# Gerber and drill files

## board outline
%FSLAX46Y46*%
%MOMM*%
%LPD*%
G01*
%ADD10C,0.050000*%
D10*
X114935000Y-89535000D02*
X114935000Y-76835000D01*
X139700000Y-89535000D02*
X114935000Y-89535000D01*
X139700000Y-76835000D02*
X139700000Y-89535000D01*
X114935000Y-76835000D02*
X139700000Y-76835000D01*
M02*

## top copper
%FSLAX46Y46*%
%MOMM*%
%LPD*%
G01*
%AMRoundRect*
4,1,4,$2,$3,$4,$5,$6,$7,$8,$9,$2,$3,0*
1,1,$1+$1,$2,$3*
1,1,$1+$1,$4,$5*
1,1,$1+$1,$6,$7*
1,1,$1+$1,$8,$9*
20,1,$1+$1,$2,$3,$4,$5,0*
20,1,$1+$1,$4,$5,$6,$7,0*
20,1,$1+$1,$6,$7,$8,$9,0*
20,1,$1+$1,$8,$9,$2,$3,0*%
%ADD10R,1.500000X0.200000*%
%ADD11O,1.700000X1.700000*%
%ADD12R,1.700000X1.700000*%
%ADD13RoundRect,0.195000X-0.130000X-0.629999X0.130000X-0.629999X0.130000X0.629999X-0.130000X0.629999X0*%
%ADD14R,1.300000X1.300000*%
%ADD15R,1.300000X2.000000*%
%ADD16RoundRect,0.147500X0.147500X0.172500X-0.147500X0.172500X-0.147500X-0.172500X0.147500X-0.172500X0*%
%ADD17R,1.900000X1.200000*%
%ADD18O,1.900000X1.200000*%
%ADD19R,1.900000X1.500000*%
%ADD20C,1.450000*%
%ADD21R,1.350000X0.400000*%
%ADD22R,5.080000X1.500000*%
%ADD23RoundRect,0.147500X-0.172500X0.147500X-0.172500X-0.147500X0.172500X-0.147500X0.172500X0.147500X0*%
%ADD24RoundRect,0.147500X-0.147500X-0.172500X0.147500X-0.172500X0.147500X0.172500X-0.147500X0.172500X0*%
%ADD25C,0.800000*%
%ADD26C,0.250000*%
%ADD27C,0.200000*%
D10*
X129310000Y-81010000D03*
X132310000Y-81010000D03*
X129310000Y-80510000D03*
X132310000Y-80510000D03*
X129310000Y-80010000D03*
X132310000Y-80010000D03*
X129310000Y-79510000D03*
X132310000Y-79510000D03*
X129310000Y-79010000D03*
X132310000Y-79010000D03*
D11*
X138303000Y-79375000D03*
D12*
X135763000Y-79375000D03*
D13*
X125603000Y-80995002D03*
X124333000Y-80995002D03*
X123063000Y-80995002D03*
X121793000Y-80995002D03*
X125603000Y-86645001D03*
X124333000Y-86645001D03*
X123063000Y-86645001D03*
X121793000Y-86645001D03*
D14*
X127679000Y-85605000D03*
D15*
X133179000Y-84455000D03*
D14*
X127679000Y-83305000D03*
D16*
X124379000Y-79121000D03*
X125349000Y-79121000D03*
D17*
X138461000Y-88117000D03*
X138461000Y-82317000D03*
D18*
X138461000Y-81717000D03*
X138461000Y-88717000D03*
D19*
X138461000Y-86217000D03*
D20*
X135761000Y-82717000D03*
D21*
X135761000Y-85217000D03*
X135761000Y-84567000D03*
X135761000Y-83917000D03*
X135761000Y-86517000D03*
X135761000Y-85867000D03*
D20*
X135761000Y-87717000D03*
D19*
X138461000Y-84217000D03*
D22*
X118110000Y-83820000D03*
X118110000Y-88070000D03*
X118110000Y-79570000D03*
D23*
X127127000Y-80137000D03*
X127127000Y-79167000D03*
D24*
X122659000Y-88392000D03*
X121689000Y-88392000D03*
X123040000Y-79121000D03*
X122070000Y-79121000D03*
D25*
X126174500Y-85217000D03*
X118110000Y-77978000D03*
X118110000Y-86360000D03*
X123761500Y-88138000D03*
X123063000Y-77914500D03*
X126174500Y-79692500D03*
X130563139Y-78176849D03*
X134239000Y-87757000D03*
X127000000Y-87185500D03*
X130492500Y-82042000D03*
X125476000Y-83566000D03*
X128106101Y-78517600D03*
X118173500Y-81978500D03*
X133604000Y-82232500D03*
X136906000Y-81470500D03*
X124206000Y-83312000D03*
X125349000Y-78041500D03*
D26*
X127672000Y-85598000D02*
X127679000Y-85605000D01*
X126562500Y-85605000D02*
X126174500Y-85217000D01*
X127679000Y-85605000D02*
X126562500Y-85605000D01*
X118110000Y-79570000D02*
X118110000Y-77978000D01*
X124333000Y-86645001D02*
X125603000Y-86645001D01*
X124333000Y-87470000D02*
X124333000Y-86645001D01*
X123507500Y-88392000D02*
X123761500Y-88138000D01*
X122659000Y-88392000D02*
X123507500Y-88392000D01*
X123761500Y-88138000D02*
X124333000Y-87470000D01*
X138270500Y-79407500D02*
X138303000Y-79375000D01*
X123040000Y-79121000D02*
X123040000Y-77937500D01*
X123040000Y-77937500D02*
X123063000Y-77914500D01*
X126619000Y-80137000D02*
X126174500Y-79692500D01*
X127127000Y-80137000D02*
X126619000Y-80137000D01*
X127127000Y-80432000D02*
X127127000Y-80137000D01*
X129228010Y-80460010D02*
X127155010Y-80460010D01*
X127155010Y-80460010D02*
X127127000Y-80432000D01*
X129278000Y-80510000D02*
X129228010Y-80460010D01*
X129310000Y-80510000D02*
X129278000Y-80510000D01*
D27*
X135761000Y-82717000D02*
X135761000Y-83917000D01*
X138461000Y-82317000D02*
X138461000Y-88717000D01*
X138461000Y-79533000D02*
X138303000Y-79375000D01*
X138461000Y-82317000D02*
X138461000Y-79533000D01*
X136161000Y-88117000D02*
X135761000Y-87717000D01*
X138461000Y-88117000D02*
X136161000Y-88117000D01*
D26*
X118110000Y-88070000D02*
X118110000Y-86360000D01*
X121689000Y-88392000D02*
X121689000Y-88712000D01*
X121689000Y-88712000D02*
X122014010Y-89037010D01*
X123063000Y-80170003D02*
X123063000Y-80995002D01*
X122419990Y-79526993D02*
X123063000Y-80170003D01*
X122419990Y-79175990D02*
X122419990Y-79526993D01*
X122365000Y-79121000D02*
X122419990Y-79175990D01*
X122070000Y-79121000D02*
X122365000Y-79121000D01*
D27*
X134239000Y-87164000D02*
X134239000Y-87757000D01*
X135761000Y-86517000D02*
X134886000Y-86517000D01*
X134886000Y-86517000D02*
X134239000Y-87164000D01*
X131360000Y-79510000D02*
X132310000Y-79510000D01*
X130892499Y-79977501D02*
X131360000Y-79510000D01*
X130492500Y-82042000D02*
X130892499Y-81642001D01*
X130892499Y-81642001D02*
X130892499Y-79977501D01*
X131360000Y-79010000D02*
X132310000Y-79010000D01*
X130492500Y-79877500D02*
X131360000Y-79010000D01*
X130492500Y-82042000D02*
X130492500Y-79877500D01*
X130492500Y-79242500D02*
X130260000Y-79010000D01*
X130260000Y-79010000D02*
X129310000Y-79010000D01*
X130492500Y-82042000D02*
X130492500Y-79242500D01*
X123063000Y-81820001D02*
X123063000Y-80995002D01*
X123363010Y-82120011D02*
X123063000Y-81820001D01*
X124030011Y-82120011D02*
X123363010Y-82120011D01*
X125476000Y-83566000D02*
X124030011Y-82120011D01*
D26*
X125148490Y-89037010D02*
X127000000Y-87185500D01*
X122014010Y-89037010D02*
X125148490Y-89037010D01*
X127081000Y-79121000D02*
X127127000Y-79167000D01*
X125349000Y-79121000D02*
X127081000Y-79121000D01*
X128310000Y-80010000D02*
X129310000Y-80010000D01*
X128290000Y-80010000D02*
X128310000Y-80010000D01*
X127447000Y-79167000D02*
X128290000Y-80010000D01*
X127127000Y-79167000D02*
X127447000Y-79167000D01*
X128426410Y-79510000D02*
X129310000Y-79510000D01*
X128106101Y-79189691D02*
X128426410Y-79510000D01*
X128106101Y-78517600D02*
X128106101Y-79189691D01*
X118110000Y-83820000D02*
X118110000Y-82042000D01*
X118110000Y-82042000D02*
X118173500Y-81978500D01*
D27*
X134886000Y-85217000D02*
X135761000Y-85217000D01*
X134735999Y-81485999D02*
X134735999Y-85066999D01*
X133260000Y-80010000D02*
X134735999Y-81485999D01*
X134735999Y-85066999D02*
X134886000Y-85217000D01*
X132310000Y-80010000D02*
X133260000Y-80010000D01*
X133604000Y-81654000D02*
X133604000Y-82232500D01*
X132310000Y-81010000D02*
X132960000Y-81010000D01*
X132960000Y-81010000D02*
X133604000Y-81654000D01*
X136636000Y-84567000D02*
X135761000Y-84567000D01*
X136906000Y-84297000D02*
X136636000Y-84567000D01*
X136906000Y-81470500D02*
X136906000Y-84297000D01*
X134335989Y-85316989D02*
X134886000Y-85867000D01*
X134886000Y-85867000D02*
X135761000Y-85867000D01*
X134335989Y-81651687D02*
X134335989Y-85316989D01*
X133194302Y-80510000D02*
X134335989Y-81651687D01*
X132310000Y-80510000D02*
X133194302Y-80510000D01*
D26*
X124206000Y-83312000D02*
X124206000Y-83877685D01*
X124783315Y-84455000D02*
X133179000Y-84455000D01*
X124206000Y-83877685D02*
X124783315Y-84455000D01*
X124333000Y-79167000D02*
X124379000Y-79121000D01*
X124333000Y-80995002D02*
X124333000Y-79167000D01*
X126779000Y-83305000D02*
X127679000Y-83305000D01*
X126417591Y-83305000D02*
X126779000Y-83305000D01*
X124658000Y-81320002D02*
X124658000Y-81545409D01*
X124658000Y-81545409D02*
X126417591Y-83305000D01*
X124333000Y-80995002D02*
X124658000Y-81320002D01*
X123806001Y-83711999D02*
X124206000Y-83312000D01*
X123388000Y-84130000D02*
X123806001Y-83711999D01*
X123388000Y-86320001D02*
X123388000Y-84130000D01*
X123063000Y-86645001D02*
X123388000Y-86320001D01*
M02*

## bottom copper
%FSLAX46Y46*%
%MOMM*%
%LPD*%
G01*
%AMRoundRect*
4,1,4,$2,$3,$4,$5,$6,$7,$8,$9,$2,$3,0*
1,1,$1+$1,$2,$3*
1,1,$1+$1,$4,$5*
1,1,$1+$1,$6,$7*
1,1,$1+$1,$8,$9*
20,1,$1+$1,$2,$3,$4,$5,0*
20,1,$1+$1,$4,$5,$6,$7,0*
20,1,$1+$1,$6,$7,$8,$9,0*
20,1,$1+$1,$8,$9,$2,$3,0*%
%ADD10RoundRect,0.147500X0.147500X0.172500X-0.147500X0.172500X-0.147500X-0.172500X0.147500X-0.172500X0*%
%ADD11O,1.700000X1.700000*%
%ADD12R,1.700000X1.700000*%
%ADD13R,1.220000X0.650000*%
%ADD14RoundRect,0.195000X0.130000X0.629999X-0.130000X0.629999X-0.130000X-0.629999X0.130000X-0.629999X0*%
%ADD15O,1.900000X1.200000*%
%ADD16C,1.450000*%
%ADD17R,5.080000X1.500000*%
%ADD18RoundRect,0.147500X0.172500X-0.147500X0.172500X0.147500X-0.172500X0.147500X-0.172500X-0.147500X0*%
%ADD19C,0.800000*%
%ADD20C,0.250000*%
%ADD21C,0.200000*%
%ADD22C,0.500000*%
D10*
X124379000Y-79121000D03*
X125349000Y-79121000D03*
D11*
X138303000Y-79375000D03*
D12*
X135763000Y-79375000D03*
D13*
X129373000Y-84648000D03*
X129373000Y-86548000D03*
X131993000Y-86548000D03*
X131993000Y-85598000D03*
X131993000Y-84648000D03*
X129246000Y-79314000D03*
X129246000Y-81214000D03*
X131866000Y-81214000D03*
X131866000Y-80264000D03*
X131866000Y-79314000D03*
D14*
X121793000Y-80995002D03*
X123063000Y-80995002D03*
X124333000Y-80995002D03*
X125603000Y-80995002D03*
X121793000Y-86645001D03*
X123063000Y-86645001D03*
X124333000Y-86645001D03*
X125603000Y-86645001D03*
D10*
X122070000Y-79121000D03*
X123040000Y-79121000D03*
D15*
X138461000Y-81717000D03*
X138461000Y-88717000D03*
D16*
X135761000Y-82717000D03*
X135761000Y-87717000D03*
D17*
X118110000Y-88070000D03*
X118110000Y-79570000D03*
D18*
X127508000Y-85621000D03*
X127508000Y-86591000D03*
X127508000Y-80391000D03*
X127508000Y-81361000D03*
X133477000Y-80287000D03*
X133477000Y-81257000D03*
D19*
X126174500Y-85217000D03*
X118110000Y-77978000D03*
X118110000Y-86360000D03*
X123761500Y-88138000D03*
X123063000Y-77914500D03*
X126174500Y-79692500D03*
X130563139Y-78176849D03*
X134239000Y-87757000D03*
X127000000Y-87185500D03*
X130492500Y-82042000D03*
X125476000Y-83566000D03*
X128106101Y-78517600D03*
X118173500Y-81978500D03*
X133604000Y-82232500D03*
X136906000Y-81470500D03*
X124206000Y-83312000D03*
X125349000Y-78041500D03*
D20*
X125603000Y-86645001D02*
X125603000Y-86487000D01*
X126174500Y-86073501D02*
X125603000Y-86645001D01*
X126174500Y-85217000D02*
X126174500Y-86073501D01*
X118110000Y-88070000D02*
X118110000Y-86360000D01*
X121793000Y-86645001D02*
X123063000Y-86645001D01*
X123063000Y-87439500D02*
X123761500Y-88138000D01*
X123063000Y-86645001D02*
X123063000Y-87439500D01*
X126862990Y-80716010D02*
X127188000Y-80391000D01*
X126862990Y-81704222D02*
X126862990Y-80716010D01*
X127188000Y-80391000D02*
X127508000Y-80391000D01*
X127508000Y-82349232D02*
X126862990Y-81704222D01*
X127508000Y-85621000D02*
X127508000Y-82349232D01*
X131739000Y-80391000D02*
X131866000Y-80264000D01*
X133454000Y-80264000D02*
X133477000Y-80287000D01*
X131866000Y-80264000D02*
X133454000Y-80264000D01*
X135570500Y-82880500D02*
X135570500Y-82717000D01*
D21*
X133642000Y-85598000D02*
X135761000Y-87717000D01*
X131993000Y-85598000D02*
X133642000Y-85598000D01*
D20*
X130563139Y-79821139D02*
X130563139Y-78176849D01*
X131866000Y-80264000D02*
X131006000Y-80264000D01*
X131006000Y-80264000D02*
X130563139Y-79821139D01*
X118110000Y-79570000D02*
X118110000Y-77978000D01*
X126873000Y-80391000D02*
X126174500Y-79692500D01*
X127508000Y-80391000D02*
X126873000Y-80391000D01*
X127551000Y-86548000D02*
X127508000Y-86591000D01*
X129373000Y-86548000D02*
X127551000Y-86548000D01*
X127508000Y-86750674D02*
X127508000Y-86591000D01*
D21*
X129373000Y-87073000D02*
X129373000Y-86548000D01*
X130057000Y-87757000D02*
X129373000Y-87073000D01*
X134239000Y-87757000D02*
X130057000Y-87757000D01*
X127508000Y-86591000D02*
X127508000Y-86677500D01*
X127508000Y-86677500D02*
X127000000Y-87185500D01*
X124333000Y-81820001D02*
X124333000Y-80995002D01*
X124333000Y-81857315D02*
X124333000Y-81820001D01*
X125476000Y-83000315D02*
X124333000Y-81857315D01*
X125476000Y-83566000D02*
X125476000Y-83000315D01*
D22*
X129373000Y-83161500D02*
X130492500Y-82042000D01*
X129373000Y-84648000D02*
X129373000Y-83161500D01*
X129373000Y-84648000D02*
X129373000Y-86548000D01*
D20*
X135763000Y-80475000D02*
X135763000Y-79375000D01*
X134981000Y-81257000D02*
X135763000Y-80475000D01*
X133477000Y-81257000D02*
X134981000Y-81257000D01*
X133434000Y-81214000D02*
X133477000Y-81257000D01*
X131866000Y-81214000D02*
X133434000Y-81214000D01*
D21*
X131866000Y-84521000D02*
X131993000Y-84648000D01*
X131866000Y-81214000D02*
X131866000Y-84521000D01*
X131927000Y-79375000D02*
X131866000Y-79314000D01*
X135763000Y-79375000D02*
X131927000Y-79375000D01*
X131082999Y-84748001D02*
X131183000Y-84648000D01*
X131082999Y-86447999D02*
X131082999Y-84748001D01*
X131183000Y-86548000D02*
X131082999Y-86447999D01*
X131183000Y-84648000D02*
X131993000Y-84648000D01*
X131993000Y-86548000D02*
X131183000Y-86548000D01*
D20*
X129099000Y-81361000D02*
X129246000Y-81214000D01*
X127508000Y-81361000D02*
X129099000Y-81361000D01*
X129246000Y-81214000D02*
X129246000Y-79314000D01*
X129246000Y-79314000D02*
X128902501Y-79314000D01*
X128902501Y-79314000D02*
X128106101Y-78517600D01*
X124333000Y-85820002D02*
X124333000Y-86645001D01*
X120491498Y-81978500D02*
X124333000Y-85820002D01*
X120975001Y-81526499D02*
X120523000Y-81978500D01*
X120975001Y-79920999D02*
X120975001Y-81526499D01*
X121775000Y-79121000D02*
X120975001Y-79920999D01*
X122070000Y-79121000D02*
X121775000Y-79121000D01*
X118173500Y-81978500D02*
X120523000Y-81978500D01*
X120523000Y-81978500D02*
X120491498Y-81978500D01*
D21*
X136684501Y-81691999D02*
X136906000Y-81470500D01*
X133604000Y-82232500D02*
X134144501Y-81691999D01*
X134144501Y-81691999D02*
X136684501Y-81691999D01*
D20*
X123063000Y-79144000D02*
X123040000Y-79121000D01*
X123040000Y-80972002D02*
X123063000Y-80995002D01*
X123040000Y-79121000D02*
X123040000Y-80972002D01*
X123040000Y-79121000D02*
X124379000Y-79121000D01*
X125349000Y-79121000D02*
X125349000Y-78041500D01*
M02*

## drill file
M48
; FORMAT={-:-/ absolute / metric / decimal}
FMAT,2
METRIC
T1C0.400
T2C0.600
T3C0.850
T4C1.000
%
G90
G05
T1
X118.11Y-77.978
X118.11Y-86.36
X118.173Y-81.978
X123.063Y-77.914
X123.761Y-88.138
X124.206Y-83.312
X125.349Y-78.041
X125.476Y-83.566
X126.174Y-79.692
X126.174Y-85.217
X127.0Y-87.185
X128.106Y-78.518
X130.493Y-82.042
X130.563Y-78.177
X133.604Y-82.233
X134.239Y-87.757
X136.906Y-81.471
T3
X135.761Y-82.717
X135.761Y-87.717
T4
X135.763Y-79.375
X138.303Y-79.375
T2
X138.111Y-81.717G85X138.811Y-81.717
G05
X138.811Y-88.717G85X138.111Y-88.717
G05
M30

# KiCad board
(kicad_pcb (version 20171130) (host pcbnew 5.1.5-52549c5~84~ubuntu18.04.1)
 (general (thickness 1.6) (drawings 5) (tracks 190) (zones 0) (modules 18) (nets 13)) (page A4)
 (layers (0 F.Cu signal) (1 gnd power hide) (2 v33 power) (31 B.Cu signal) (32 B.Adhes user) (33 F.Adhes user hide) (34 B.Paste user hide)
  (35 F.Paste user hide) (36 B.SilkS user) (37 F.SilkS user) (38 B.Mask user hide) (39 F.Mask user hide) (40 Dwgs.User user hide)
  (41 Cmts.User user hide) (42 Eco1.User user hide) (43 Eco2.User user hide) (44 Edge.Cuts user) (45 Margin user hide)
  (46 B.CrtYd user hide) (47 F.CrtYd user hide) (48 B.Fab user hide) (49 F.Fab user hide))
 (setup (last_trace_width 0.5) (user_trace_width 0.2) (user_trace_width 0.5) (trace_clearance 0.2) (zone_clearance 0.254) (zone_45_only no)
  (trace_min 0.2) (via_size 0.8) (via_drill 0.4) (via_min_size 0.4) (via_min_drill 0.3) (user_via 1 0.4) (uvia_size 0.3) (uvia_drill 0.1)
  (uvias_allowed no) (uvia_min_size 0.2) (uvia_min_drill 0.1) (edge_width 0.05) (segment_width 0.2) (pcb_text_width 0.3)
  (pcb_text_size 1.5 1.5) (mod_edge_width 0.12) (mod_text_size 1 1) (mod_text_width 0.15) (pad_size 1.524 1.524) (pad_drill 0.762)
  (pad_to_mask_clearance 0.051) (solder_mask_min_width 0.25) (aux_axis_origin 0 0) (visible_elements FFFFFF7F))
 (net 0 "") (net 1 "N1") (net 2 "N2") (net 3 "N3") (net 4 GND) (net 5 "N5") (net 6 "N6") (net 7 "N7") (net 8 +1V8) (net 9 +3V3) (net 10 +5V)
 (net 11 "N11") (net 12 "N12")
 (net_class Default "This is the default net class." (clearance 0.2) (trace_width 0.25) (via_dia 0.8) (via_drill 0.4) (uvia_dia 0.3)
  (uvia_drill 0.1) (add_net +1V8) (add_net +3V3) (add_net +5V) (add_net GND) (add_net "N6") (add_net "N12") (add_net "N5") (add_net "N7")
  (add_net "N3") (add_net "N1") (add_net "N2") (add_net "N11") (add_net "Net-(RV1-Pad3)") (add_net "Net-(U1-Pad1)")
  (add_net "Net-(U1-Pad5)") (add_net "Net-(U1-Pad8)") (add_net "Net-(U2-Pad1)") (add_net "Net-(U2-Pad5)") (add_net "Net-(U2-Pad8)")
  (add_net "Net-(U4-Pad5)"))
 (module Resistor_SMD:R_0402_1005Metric (layer B.Cu) (at 124.864 79.121 180)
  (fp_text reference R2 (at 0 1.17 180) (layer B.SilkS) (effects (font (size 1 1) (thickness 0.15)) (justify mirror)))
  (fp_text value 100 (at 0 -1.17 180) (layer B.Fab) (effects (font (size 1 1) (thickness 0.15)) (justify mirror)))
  (pad 2 smd roundrect (at 0.485 0 180) (size 0.59 0.64) (layers B.Cu B.Paste B.Mask) (roundrect_rratio 0.25) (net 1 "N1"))
  (pad 1 smd roundrect (at -0.485 0 180) (size 0.59 0.64) (layers B.Cu B.Paste B.Mask) (roundrect_rratio 0.25) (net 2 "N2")))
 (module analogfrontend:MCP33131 (layer F.Cu) (at 130.81 80.01 270)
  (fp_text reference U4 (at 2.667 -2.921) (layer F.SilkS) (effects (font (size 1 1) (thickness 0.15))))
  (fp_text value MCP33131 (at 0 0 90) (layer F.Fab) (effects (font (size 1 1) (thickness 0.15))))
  (pad 5 smd rect (at 1 1.5 270) (size 0.2 1.5) (layers F.Cu F.Paste F.Mask))
  (pad 6 smd rect (at 1 -1.5 270) (size 0.2 1.5) (layers F.Cu F.Paste F.Mask) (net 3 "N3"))
  (pad 4 smd rect (at 0.5 1.5 270) (size 0.2 1.5) (layers F.Cu F.Paste F.Mask) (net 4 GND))
  (pad 7 smd rect (at 0.5 -1.5 270) (size 0.2 1.5) (layers F.Cu F.Paste F.Mask) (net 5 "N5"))
  (pad 3 smd rect (at 0 1.5 270) (size 0.2 1.5) (layers F.Cu F.Paste F.Mask) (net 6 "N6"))
  (pad 8 smd rect (at 0 -1.5 270) (size 0.2 1.5) (layers F.Cu F.Paste F.Mask) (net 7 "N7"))
  (pad 2 smd rect (at -0.5 1.5 270) (size 0.2 1.5) (layers F.Cu F.Paste F.Mask) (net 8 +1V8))
  (pad 9 smd rect (at -0.5 -1.5 270) (size 0.2 1.5) (layers F.Cu F.Paste F.Mask) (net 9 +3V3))
  (pad 1 smd rect (at -1 1.5 270) (size 0.2 1.5) (layers F.Cu F.Paste F.Mask) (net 9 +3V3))
  (pad 10 smd rect (at -1 -1.5 270) (size 0.2 1.5) (layers F.Cu F.Paste F.Mask) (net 9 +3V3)))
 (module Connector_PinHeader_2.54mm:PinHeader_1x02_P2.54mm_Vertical (layer F.Cu) (at 135.763 79.375 90)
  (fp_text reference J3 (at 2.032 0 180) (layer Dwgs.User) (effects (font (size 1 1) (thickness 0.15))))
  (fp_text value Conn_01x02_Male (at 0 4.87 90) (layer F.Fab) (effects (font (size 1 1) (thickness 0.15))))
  (pad 2 thru_hole oval (at 0 2.54 90) (size 1.7 1.7) (drill 1) (layers *.Cu *.Mask) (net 4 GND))
  (pad 1 thru_hole rect (at 0 0 90) (size 1.7 1.7) (drill 1) (layers *.Cu *.Mask) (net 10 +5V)))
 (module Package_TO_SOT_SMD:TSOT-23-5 (layer B.Cu) (at 130.683 85.598 180)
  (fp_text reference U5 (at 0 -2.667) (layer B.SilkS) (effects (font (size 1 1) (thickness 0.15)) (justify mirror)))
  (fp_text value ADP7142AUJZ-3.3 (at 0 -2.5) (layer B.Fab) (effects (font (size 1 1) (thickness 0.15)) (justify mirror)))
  (pad 5 smd rect (at 1.31 0.95 180) (size 1.22 0.65) (layers B.Cu B.Paste B.Mask) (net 9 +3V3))
  (pad 4 smd rect (at 1.31 -0.95 180) (size 1.22 0.65) (layers B.Cu B.Paste B.Mask) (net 9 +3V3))
  (pad 3 smd rect (at -1.31 -0.95 180) (size 1.22 0.65) (layers B.Cu B.Paste B.Mask) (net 10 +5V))
  (pad 2 smd rect (at -1.31 0 180) (size 1.22 0.65) (layers B.Cu B.Paste B.Mask) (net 4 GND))
  (pad 1 smd rect (at -1.31 0.95 180) (size 1.22 0.65) (layers B.Cu B.Paste B.Mask) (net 10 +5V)))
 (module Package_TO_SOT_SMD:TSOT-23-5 (layer B.Cu) (at 130.556 80.264 180)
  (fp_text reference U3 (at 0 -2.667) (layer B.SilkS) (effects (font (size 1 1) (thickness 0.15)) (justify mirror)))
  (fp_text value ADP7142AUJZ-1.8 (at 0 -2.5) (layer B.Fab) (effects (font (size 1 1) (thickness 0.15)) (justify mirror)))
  (pad 5 smd rect (at 1.31 0.95 180) (size 1.22 0.65) (layers B.Cu B.Paste B.Mask) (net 8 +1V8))
  (pad 4 smd rect (at 1.31 -0.95 180) (size 1.22 0.65) (layers B.Cu B.Paste B.Mask) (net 8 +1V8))
  (pad 3 smd rect (at -1.31 -0.95 180) (size 1.22 0.65) (layers B.Cu B.Paste B.Mask) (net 10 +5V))
  (pad 2 smd rect (at -1.31 0 180) (size 1.22 0.65) (layers B.Cu B.Paste B.Mask) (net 4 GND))
  (pad 1 smd rect (at -1.31 0.95 180) (size 1.22 0.65) (layers B.Cu B.Paste B.Mask) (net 10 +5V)))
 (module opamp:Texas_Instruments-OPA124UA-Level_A (layer F.Cu) (at 123.698 83.82 90)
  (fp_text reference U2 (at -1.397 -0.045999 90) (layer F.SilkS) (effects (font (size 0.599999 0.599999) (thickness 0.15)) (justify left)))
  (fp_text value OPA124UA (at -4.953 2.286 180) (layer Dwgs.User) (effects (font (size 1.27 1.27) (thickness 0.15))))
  (pad 5 smd roundrect (at 2.824998 1.905) (size 0.650001 1.649999) (layers F.Cu F.Paste F.Mask) (roundrect_rratio 0.2999995385))
  (pad 6 smd roundrect (at 2.824998 0.635) (size 0.650001 1.649999) (layers F.Cu F.Paste F.Mask) (roundrect_rratio 0.2999995385)
   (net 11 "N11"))
  (pad 7 smd roundrect (at 2.824998 -0.635) (size 0.650001 1.649999) (layers F.Cu F.Paste F.Mask) (roundrect_rratio 0.2999995385)
   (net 9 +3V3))
  (pad 8 smd roundrect (at 2.824998 -1.905) (size 0.650001 1.649999) (layers F.Cu F.Paste F.Mask) (roundrect_rratio 0.2999995385))
  (pad 4 smd roundrect (at -2.825001 1.905) (size 0.650001 1.649999) (layers F.Cu F.Paste F.Mask) (roundrect_rratio 0.2999995385)
   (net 4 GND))
  (pad 3 smd roundrect (at -2.825001 0.635) (size 0.650001 1.649999) (layers F.Cu F.Paste F.Mask) (roundrect_rratio 0.2999995385)
   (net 4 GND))
  (pad 2 smd roundrect (at -2.825001 -0.635) (size 0.650001 1.649999) (layers F.Cu F.Paste F.Mask) (roundrect_rratio 0.2999995385)
   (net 2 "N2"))
  (pad 1 smd roundrect (at -2.825001 -1.905) (size 0.650001 1.649999) (layers F.Cu F.Paste F.Mask) (roundrect_rratio 0.2999995385)))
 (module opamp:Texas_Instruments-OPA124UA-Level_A (layer B.Cu) (at 123.698 83.82 90)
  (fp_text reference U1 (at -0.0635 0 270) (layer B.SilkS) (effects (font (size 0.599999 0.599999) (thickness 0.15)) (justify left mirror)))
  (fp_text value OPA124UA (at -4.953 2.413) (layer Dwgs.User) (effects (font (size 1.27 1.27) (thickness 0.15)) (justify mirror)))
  (pad 5 smd roundrect (at 2.824998 -1.905 180) (size 0.650001 1.649999) (layers B.Cu B.Paste B.Mask) (roundrect_rratio 0.2999995385))
  (pad 6 smd roundrect (at 2.824998 -0.635 180) (size 0.650001 1.649999) (layers B.Cu B.Paste B.Mask) (roundrect_rratio 0.2999995385)
   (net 1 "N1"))
  (pad 7 smd roundrect (at 2.824998 0.635 180) (size 0.650001 1.649999) (layers B.Cu B.Paste B.Mask) (roundrect_rratio 0.2999995385)
   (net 9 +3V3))
  (pad 8 smd roundrect (at 2.824998 1.905 180) (size 0.650001 1.649999) (layers B.Cu B.Paste B.Mask) (roundrect_rratio 0.2999995385))
  (pad 4 smd roundrect (at -2.825001 -1.905 180) (size 0.650001 1.649999) (layers B.Cu B.Paste B.Mask) (roundrect_rratio 0.2999995385)
   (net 4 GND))
  (pad 3 smd roundrect (at -2.825001 -0.635 180) (size 0.650001 1.649999) (layers B.Cu B.Paste B.Mask) (roundrect_rratio 0.2999995385)
   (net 4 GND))
  (pad 2 smd roundrect (at -2.825001 0.635 180) (size 0.650001 1.649999) (layers B.Cu B.Paste B.Mask) (roundrect_rratio 0.2999995385)
   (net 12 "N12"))
  (pad 1 smd roundrect (at -2.825001 1.905 180) (size 0.650001 1.649999) (layers B.Cu B.Paste B.Mask) (roundrect_rratio 0.2999995385)))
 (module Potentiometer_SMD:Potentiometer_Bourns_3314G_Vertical (layer F.Cu) (at 130.429 84.455 90)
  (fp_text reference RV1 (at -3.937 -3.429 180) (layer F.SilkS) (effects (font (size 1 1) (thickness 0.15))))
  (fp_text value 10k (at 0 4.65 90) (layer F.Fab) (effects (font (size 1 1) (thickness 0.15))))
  (pad 3 smd rect (at -1.15 -2.75 90) (size 1.3 1.3) (layers F.Cu F.Paste F.Mask))
  (pad 2 smd rect (at 0 2.75 90) (size 2 1.3) (layers F.Cu F.Paste F.Mask) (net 2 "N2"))
  (pad 1 smd rect (at 1.15 -2.75 90) (size 1.3 1.3) (layers F.Cu F.Paste F.Mask) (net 11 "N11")))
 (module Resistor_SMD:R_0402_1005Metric (layer F.Cu) (at 124.864 79.121 180)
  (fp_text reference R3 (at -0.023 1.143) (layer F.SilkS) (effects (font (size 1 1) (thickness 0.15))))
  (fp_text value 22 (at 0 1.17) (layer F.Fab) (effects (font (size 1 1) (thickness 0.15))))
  (pad 2 smd roundrect (at 0.485 0 180) (size 0.59 0.64) (layers F.Cu F.Paste F.Mask) (roundrect_rratio 0.25) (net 11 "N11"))
  (pad 1 smd roundrect (at -0.485 0 180) (size 0.59 0.64) (layers F.Cu F.Paste F.Mask) (roundrect_rratio 0.25) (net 6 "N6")))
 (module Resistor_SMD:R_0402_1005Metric (layer B.Cu) (at 122.555 79.121 180)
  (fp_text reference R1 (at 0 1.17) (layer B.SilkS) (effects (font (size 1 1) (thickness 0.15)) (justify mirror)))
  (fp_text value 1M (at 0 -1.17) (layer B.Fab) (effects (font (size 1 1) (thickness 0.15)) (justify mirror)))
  (pad 2 smd roundrect (at 0.485 0 180) (size 0.59 0.64) (layers B.Cu B.Paste B.Mask) (roundrect_rratio 0.25) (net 12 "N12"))
  (pad 1 smd roundrect (at -0.485 0 180) (size 0.59 0.64) (layers B.Cu B.Paste B.Mask) (roundrect_rratio 0.25) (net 1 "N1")))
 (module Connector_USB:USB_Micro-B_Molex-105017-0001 (layer F.Cu) (at 137.2235 85.217 90)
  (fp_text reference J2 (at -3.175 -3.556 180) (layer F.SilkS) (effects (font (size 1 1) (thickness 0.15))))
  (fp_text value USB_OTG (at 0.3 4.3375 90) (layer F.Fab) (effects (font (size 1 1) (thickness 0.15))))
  (pad 6 smd rect (at -2.9 1.2375 90) (size 1.2 1.9) (layers F.Cu F.Mask) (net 4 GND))
  (pad 6 smd rect (at 2.9 1.2375 90) (size 1.2 1.9) (layers F.Cu F.Mask) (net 4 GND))
  (pad 6 thru_hole oval (at 3.5 1.2375 90) (size 1.2 1.9) (drill oval 0.6 1.3) (layers *.Cu *.Mask) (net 4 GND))
  (pad 6 thru_hole oval (at -3.5 1.2375 270) (size 1.2 1.9) (drill oval 0.6 1.3) (layers *.Cu *.Mask) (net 4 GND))
  (pad 6 smd rect (at -1 1.2375 90) (size 1.5 1.9) (layers F.Cu F.Paste F.Mask) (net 4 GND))
  (pad 6 thru_hole circle (at 2.5 -1.4625 90) (size 1.45 1.45) (drill 0.85) (layers *.Cu *.Mask) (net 4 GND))
  (pad 3 smd rect (at 0 -1.4625 90) (size 0.4 1.35) (layers F.Cu F.Paste F.Mask) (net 7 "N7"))
  (pad 4 smd rect (at 0.65 -1.4625 90) (size 0.4 1.35) (layers F.Cu F.Paste F.Mask) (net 3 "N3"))
  (pad 5 smd rect (at 1.3 -1.4625 90) (size 0.4 1.35) (layers F.Cu F.Paste F.Mask) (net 4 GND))
  (pad 1 smd rect (at -1.3 -1.4625 90) (size 0.4 1.35) (layers F.Cu F.Paste F.Mask) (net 9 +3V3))
  (pad 2 smd rect (at -0.65 -1.4625 90) (size 0.4 1.35) (layers F.Cu F.Paste F.Mask) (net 5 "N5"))
  (pad 6 thru_hole circle (at -2.5 -1.4625 90) (size 1.45 1.45) (drill 0.85) (layers *.Cu *.Mask) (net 4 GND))
  (pad 6 smd rect (at 1 1.2375 90) (size 1.5 1.9) (layers F.Cu F.Paste F.Mask) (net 4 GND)))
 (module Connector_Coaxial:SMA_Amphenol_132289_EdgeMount (layer F.Cu) (at 118.11 83.82 180)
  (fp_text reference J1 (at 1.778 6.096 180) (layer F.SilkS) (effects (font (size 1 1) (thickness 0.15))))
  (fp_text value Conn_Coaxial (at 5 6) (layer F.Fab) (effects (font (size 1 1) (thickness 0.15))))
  (pad 1 smd rect (at 0 0 270) (size 1.5 5.08) (layers F.Cu F.Paste F.Mask) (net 12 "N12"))
  (pad 2 smd rect (at 0 -4.25 270) (size 1.5 5.08) (layers F.Cu F.Paste F.Mask) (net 4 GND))
  (pad 2 smd rect (at 0 4.25 270) (size 1.5 5.08) (layers F.Cu F.Paste F.Mask) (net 4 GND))
  (pad 2 smd rect (at 0 -4.25 270) (size 1.5 5.08) (layers B.Cu B.Paste B.Mask) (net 4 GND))
  (pad 2 smd rect (at 0 4.25 270) (size 1.5 5.08) (layers B.Cu B.Paste B.Mask) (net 4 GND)))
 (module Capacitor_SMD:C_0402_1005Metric (layer B.Cu) (at 127.508 86.106 90)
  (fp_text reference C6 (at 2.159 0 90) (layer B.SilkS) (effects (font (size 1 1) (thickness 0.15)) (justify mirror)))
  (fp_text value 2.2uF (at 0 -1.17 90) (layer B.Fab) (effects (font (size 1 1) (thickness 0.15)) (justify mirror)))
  (pad 2 smd roundrect (at 0.485 0 90) (size 0.59 0.64) (layers B.Cu B.Paste B.Mask) (roundrect_rratio 0.25) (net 4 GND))
  (pad 1 smd roundrect (at -0.485 0 90) (size 0.59 0.64) (layers B.Cu B.Paste B.Mask) (roundrect_rratio 0.25) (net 9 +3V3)))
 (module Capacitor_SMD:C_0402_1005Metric (layer B.Cu) (at 127.508 80.876 90)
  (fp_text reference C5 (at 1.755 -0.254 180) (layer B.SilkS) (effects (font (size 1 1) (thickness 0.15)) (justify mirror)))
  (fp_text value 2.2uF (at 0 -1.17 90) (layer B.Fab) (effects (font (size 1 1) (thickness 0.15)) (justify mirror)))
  (pad 2 smd roundrect (at 0.485 0 90) (size 0.59 0.64) (layers B.Cu B.Paste B.Mask) (roundrect_rratio 0.25) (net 4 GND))
  (pad 1 smd roundrect (at -0.485 0 90) (size 0.59 0.64) (layers B.Cu B.Paste B.Mask) (roundrect_rratio 0.25) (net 8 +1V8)))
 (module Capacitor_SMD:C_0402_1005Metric (layer F.Cu) (at 127.127 79.652 270)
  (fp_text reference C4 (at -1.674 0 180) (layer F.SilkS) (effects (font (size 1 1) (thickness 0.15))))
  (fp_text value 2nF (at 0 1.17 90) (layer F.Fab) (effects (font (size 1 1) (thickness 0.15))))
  (pad 2 smd roundrect (at 0.485 0 270) (size 0.59 0.64) (layers F.Cu F.Paste F.Mask) (roundrect_rratio 0.25) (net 4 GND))
  (pad 1 smd roundrect (at -0.485 0 270) (size 0.59 0.64) (layers F.Cu F.Paste F.Mask) (roundrect_rratio 0.25) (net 6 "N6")))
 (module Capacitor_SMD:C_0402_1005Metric (layer B.Cu) (at 133.477 80.772 90)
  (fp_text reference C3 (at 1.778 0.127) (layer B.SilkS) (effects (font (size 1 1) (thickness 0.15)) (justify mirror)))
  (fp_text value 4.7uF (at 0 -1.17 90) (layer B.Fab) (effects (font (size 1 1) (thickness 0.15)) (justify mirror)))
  (pad 2 smd roundrect (at 0.485 0 90) (size 0.59 0.64) (layers B.Cu B.Paste B.Mask) (roundrect_rratio 0.25) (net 4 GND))
  (pad 1 smd roundrect (at -0.485 0 90) (size 0.59 0.64) (layers B.Cu B.Paste B.Mask) (roundrect_rratio 0.25) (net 10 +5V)))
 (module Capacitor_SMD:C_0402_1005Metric (layer F.Cu) (at 122.174 88.392)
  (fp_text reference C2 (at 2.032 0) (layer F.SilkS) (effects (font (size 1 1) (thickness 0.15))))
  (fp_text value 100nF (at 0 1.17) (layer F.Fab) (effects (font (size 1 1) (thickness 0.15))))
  (pad 2 smd roundrect (at 0.485 0) (size 0.59 0.64) (layers F.Cu F.Paste F.Mask) (roundrect_rratio 0.25) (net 4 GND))
  (pad 1 smd roundrect (at -0.485 0) (size 0.59 0.64) (layers F.Cu F.Paste F.Mask) (roundrect_rratio 0.25) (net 9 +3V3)))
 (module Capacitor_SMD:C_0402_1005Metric (layer F.Cu) (at 122.555 79.121)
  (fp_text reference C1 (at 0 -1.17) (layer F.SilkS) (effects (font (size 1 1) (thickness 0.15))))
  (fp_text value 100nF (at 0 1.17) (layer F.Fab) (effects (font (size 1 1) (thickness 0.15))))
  (pad 2 smd roundrect (at 0.485 0) (size 0.59 0.64) (layers F.Cu F.Paste F.Mask) (roundrect_rratio 0.25) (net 4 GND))
  (pad 1 smd roundrect (at -0.485 0) (size 0.59 0.64) (layers F.Cu F.Paste F.Mask) (roundrect_rratio 0.25) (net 9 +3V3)))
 (gr_line (start 114.935 89.535) (end 114.935 76.835) (layer Edge.Cuts) (width 0.05))
 (gr_line (start 139.7 89.535) (end 114.935 89.535) (layer Edge.Cuts) (width 0.05))
 (gr_line (start 139.7 76.835) (end 139.7 89.535) (layer Edge.Cuts) (width 0.05))
 (gr_line (start 114.935 76.835) (end 139.7 76.835) (layer Edge.Cuts) (width 0.05))
 (via (at 126.1745 85.217) (size 0.8) (drill 0.4) (layers F.Cu B.Cu) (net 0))
 (segment (start 125.603 86.645001) (end 125.603 86.487) (width 0.25) (layer B.Cu) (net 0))
 (segment (start 127.672 85.598) (end 127.679 85.605) (width 0.25) (layer F.Cu) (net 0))
 (segment (start 126.5625 85.605) (end 126.1745 85.217) (width 0.25) (layer F.Cu) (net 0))
 (segment (start 127.679 85.605) (end 126.5625 85.605) (width 0.25) (layer F.Cu) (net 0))
 (segment (start 126.1745 86.073501) (end 125.603 86.645001) (width 0.25) (layer B.Cu) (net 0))
 (segment (start 126.1745 85.217) (end 126.1745 86.073501) (width 0.25) (layer B.Cu) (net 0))
 (via (at 118.11 77.978) (size 0.8) (drill 0.4) (layers F.Cu B.Cu) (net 4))
 (segment (start 118.11 79.57) (end 118.11 77.978) (width 0.25) (layer F.Cu) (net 4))
 (via (at 118.11 86.36) (size 0.8) (drill 0.4) (layers F.Cu B.Cu) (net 4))
 (segment (start 118.11 88.07) (end 118.11 86.36) (width 0.25) (layer B.Cu) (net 4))
 (segment (start 124.333 86.645001) (end 125.603 86.645001) (width 0.25) (layer F.Cu) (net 4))
 (segment (start 124.333 87.47) (end 124.333 86.645001) (width 0.25) (layer F.Cu) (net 4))
 (via (at 123.7615 88.138) (size 0.8) (drill 0.4) (layers F.Cu B.Cu) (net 4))
 (segment (start 123.5075 88.392) (end 123.7615 88.138) (width 0.25) (layer F.Cu) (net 4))
 (segment (start 122.659 88.392) (end 123.5075 88.392) (width 0.25) (layer F.Cu) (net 4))
 (segment (start 123.7615 88.138) (end 124.333 87.47) (width 0.25) (layer F.Cu) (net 4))
 (segment (start 121.793 86.645001) (end 123.063 86.645001) (width 0.25) (layer B.Cu) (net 4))
 (segment (start 123.063 87.4395) (end 123.7615 88.138) (width 0.25) (layer B.Cu) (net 4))
 (segment (start 123.063 86.645001) (end 123.063 87.4395) (width 0.25) (layer B.Cu) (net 4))
 (segment (start 138.2705 79.4075) (end 138.303 79.375) (width 0.25) (layer F.Cu) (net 4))
 (segment (start 126.86299 80.71601) (end 127.188 80.391) (width 0.25) (layer B.Cu) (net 4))
 (segment (start 126.86299 81.704222) (end 126.86299 80.71601) (width 0.25) (layer B.Cu) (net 4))
 (segment (start 127.188 80.391) (end 127.508 80.391) (width 0.25) (layer B.Cu) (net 4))
 (segment (start 127.508 82.349232) (end 126.86299 81.704222) (width 0.25) (layer B.Cu) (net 4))
 (segment (start 127.508 85.621) (end 127.508 82.349232) (width 0.25) (layer B.Cu) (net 4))
 (via (at 123.063 77.9145) (size 0.8) (drill 0.4) (layers F.Cu B.Cu) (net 4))
 (segment (start 123.04 79.121) (end 123.04 77.9375) (width 0.25) (layer F.Cu) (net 4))
 (segment (start 123.04 77.9375) (end 123.063 77.9145) (width 0.25) (layer F.Cu) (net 4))
 (segment (start 123.628685 77.9145) (end 125.914685 80.2005) (width 0.25) (layer gnd) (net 4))
 (segment (start 123.063 77.9145) (end 123.628685 77.9145) (width 0.25) (layer gnd) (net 4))
 (via (at 126.1745 79.6925) (size 0.8) (drill 0.4) (layers F.Cu B.Cu) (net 4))
 (segment (start 126.619 80.137) (end 126.1745 79.6925) (width 0.25) (layer F.Cu) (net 4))
 (segment (start 127.127 80.137) (end 126.619 80.137) (width 0.25) (layer F.Cu) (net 4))
 (segment (start 131.739 80.391) (end 131.866 80.264) (width 0.25) (layer B.Cu) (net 4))
 (segment (start 133.454 80.264) (end 133.477 80.287) (width 0.25) (layer B.Cu) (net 4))
 (segment (start 131.866 80.264) (end 133.454 80.264) (width 0.25) (layer B.Cu) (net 4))
 (segment (start 135.5705 82.8805) (end 135.5705 82.717) (width 0.25) (layer B.Cu) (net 4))
 (segment (start 127.127 80.432) (end 127.127 80.137) (width 0.25) (layer F.Cu) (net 4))
 (segment (start 129.22801 80.46001) (end 127.15501 80.46001) (width 0.25) (layer F.Cu) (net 4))
 (segment (start 127.15501 80.46001) (end 127.127 80.432) (width 0.25) (layer F.Cu) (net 4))
 (segment (start 129.278 80.51) (end 129.22801 80.46001) (width 0.25) (layer F.Cu) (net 4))
 (segment (start 129.31 80.51) (end 129.278 80.51) (width 0.25) (layer F.Cu) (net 4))
 (segment (start 135.761 82.717) (end 135.761 83.917) (width 0.2) (layer F.Cu) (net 4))
 (segment (start 138.461 82.317) (end 138.461 88.717) (width 0.2) (layer F.Cu) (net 4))
 (segment (start 138.461 79.533) (end 138.303 79.375) (width 0.2) (layer F.Cu) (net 4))
 (segment (start 138.461 82.317) (end 138.461 79.533) (width 0.2) (layer F.Cu) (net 4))
 (segment (start 136.161 88.117) (end 135.761 87.717) (width 0.2) (layer F.Cu) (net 4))
 (segment (start 138.461 88.117) (end 136.161 88.117) (width 0.2) (layer F.Cu) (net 4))
 (segment (start 133.642 85.598) (end 135.761 87.717) (width 0.2) (layer B.Cu) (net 4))
 (segment (start 131.993 85.598) (end 133.642 85.598) (width 0.2) (layer B.Cu) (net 4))
 (segment (start 130.563139 79.821139) (end 130.563139 78.176849) (width 0.25) (layer B.Cu) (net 4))
 (segment (start 131.866 80.264) (end 131.006 80.264) (width 0.25) (layer B.Cu) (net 4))
 (via (at 130.563139 78.176849) (size 0.8) (drill 0.4) (layers F.Cu B.Cu) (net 4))
 (segment (start 131.006 80.264) (end 130.563139 79.821139) (width 0.25) (layer B.Cu) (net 4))
 (segment (start 118.11 79.57) (end 118.11 77.978) (width 0.25) (layer B.Cu) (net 4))
 (segment (start 118.11 88.07) (end 118.11 86.36) (width 0.25) (layer F.Cu) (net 4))
 (segment (start 126.873 80.391) (end 126.1745 79.6925) (width 0.25) (layer B.Cu) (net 4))
 (segment (start 127.508 80.391) (end 126.873 80.391) (width 0.25) (layer B.Cu) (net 4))
 (segment (start 127.551 86.548) (end 127.508 86.591) (width 0.25) (layer B.Cu) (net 9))
 (segment (start 129.373 86.548) (end 127.551 86.548) (width 0.25) (layer B.Cu) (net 9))
 (segment (start 121.689 88.392) (end 121.689 88.712) (width 0.25) (layer F.Cu) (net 9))
 (segment (start 121.689 88.712) (end 122.01401 89.03701) (width 0.25) (layer F.Cu) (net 9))
 (segment (start 127.508 86.750674) (end 127.508 86.591) (width 0.25) (layer B.Cu) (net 9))
 (segment (start 123.063 80.170003) (end 123.063 80.995002) (width 0.25) (layer F.Cu) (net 9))
 (segment (start 122.41999 79.526993) (end 123.063 80.170003) (width 0.25) (layer F.Cu) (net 9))
 (segment (start 122.41999 79.17599) (end 122.41999 79.526993) (width 0.25) (layer F.Cu) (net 9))
 (segment (start 122.365 79.121) (end 122.41999 79.17599) (width 0.25) (layer F.Cu) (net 9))
 (segment (start 122.07 79.121) (end 122.365 79.121) (width 0.25) (layer F.Cu) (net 9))
 (via (at 134.239 87.757) (size 0.8) (drill 0.4) (layers F.Cu B.Cu) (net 9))
 (segment (start 134.239 87.164) (end 134.239 87.757) (width 0.2) (layer F.Cu) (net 9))
 (segment (start 135.761 86.517) (end 134.886 86.517) (width 0.2) (layer F.Cu) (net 9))
 (segment (start 134.886 86.517) (end 134.239 87.164) (width 0.2) (layer F.Cu) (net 9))
 (segment (start 129.373 87.073) (end 129.373 86.548) (width 0.2) (layer B.Cu) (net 9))
 (segment (start 130.057 87.757) (end 129.373 87.073) (width 0.2) (layer B.Cu) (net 9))
 (segment (start 134.239 87.757) (end 130.057 87.757) (width 0.2) (layer B.Cu) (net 9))
 (via (at 127 87.1855) (size 0.8) (drill 0.4) (layers F.Cu B.Cu) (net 9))
 (segment (start 127.508 86.591) (end 127.508 86.6775) (width 0.2) (layer B.Cu) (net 9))
 (segment (start 127.508 86.6775) (end 127 87.1855) (width 0.2) (layer B.Cu) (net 9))
 (via (at 130.4925 82.042) (size 0.8) (drill 0.4) (layers F.Cu B.Cu) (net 9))
 (segment (start 131.36 79.51) (end 132.31 79.51) (width 0.2) (layer F.Cu) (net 9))
 (segment (start 130.892499 79.977501) (end 131.36 79.51) (width 0.2) (layer F.Cu) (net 9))
 (segment (start 130.4925 82.042) (end 130.892499 81.642001) (width 0.2) (layer F.Cu) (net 9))
 (segment (start 130.892499 81.642001) (end 130.892499 79.977501) (width 0.2) (layer F.Cu) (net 9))
 (segment (start 131.36 79.01) (end 132.31 79.01) (width 0.2) (layer F.Cu) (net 9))
 (segment (start 130.4925 79.8775) (end 131.36 79.01) (width 0.2) (layer F.Cu) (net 9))
 (segment (start 130.4925 82.042) (end 130.4925 79.8775) (width 0.2) (layer F.Cu) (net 9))
 (segment (start 130.4925 79.2425) (end 130.26 79.01) (width 0.2) (layer F.Cu) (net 9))
 (segment (start 130.26 79.01) (end 129.31 79.01) (width 0.2) (layer F.Cu) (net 9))
 (segment (start 130.4925 82.042) (end 130.4925 79.2425) (width 0.2) (layer F.Cu) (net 9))
 (via (at 125.476 83.566) (size 0.8) (drill 0.4) (layers F.Cu B.Cu) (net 9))
 (segment (start 123.063 81.820001) (end 123.063 80.995002) (width 0.2) (layer F.Cu) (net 9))
 (segment (start 123.36301 82.120011) (end 123.063 81.820001) (width 0.2) (layer F.Cu) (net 9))
 (segment (start 124.030011 82.120011) (end 123.36301 82.120011) (width 0.2) (layer F.Cu) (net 9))
 (segment (start 125.476 83.566) (end 124.030011 82.120011) (width 0.2) (layer F.Cu) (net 9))
 (segment (start 124.333 81.820001) (end 124.333 80.995002) (width 0.2) (layer B.Cu) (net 9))
 (segment (start 124.333 81.857315) (end 124.333 81.820001) (width 0.2) (layer B.Cu) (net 9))
 (segment (start 125.476 83.000315) (end 124.333 81.857315) (width 0.2) (layer B.Cu) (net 9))
 (segment (start 125.476 83.566) (end 125.476 83.000315) (width 0.2) (layer B.Cu) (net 9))
 (segment (start 129.373 83.1615) (end 130.4925 82.042) (width 0.5) (layer B.Cu) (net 9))
 (segment (start 129.373 84.648) (end 129.373 83.1615) (width 0.5) (layer B.Cu) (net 9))
 (segment (start 129.373 84.648) (end 129.373 86.548) (width 0.5) (layer B.Cu) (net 9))
 (segment (start 125.14849 89.03701) (end 127 87.1855) (width 0.25) (layer F.Cu) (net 9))
 (segment (start 122.01401 89.03701) (end 125.14849 89.03701) (width 0.25) (layer F.Cu) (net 9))
 (segment (start 128.9685 83.566) (end 130.4925 82.042) (width 0.5) (layer v33) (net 9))
 (segment (start 125.476 83.566) (end 128.9685 83.566) (width 0.5) (layer v33) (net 9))
 (segment (start 135.763 80.475) (end 135.763 79.375) (width 0.25) (layer B.Cu) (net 10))
 (segment (start 134.981 81.257) (end 135.763 80.475) (width 0.25) (layer B.Cu) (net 10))
 (segment (start 133.477 81.257) (end 134.981 81.257) (width 0.25) (layer B.Cu) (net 10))
 (segment (start 133.434 81.214) (end 133.477 81.257) (width 0.25) (layer B.Cu) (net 10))
 (segment (start 131.866 81.214) (end 133.434 81.214) (width 0.25) (layer B.Cu) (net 10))
 (segment (start 131.866 84.521) (end 131.993 84.648) (width 0.2) (layer B.Cu) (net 10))
 (segment (start 131.866 81.214) (end 131.866 84.521) (width 0.2) (layer B.Cu) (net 10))
 (segment (start 131.927 79.375) (end 131.866 79.314) (width 0.2) (layer B.Cu) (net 10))
 (segment (start 135.763 79.375) (end 131.927 79.375) (width 0.2) (layer B.Cu) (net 10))
 (segment (start 131.082999 84.748001) (end 131.183 84.648) (width 0.2) (layer B.Cu) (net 10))
 (segment (start 131.082999 86.447999) (end 131.082999 84.748001) (width 0.2) (layer B.Cu) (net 10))
 (segment (start 131.183 86.548) (end 131.082999 86.447999) (width 0.2) (layer B.Cu) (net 10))
 (segment (start 131.183 84.648) (end 131.993 84.648) (width 0.2) (layer B.Cu) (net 10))
 (segment (start 131.993 86.548) (end 131.183 86.548) (width 0.2) (layer B.Cu) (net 10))
 (segment (start 127.081 79.121) (end 127.127 79.167) (width 0.25) (layer F.Cu) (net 6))
 (segment (start 125.349 79.121) (end 127.081 79.121) (width 0.25) (layer F.Cu) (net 6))
 (segment (start 128.31 80.01) (end 129.31 80.01) (width 0.25) (layer F.Cu) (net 6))
 (segment (start 128.29 80.01) (end 128.31 80.01) (width 0.25) (layer F.Cu) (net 6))
 (segment (start 127.447 79.167) (end 128.29 80.01) (width 0.25) (layer F.Cu) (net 6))
 (segment (start 127.127 79.167) (end 127.447 79.167) (width 0.25) (layer F.Cu) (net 6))
 (segment (start 129.099 81.361) (end 129.246 81.214) (width 0.25) (layer B.Cu) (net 8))
 (segment (start 127.508 81.361) (end 129.099 81.361) (width 0.25) (layer B.Cu) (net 8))
 (segment (start 129.246 81.214) (end 129.246 79.314) (width 0.25) (layer B.Cu) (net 8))
 (via (at 128.106101 78.5176) (size 0.8) (drill 0.4) (layers F.Cu B.Cu) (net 8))
 (segment (start 129.246 79.314) (end 128.902501 79.314) (width 0.25) (layer B.Cu) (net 8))
 (segment (start 128.902501 79.314) (end 128.106101 78.5176) (width 0.25) (layer B.Cu) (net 8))
 (segment (start 128.42641 79.51) (end 129.31 79.51) (width 0.25) (layer F.Cu) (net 8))
 (segment (start 128.106101 79.189691) (end 128.42641 79.51) (width 0.25) (layer F.Cu) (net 8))
 (segment (start 128.106101 78.5176) (end 128.106101 79.189691) (width 0.25) (layer F.Cu) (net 8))
 (via (at 118.1735 81.9785) (size 0.8) (drill 0.4) (layers F.Cu B.Cu) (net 12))
 (segment (start 118.11 83.82) (end 118.11 82.042) (width 0.25) (layer F.Cu) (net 12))
 (segment (start 118.11 82.042) (end 118.1735 81.9785) (width 0.25) (layer F.Cu) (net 12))
 (segment (start 124.333 85.820002) (end 124.333 86.645001) (width 0.25) (layer B.Cu) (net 12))
 (segment (start 120.491498 81.9785) (end 124.333 85.820002) (width 0.25) (layer B.Cu) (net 12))
 (segment (start 120.975001 81.526499) (end 120.523 81.9785) (width 0.25) (layer B.Cu) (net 12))
 (segment (start 120.975001 79.920999) (end 120.975001 81.526499) (width 0.25) (layer B.Cu) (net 12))
 (segment (start 121.775 79.121) (end 120.975001 79.920999) (width 0.25) (layer B.Cu) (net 12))
 (segment (start 122.07 79.121) (end 121.775 79.121) (width 0.25) (layer B.Cu) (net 12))
 (segment (start 118.1735 81.9785) (end 120.523 81.9785) (width 0.25) (layer B.Cu) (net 12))
 (segment (start 120.523 81.9785) (end 120.491498 81.9785) (width 0.25) (layer B.Cu) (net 12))
 (segment (start 134.886 85.217) (end 135.761 85.217) (width 0.2) (layer F.Cu) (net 7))
 (segment (start 134.735999 81.485999) (end 134.735999 85.066999) (width 0.2) (layer F.Cu) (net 7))
 (segment (start 133.26 80.01) (end 134.735999 81.485999) (width 0.2) (layer F.Cu) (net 7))
 (segment (start 134.735999 85.066999) (end 134.886 85.217) (width 0.2) (layer F.Cu) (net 7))
 (segment (start 132.31 80.01) (end 133.26 80.01) (width 0.2) (layer F.Cu) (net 7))
 (via (at 133.604 82.2325) (size 0.8) (drill 0.4) (layers F.Cu B.Cu) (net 3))
 (segment (start 133.604 81.654) (end 133.604 82.2325) (width 0.2) (layer F.Cu) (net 3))
 (segment (start 132.31 81.01) (end 132.96 81.01) (width 0.2) (layer F.Cu) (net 3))
 (segment (start 132.96 81.01) (end 133.604 81.654) (width 0.2) (layer F.Cu) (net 3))
 (via (at 136.906 81.4705) (size 0.8) (drill 0.4) (layers F.Cu B.Cu) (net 3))
 (segment (start 136.684501 81.691999) (end 136.906 81.4705) (width 0.2) (layer B.Cu) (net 3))
 (segment (start 133.604 82.2325) (end 134.144501 81.691999) (width 0.2) (layer B.Cu) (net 3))
 (segment (start 134.144501 81.691999) (end 136.684501 81.691999) (width 0.2) (layer B.Cu) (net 3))
 (segment (start 136.636 84.567) (end 135.761 84.567) (width 0.2) (layer F.Cu) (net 3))
 (segment (start 136.906 84.297) (end 136.636 84.567) (width 0.2) (layer F.Cu) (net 3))
 (segment (start 136.906 81.4705) (end 136.906 84.297) (width 0.2) (layer F.Cu) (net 3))
 (segment (start 134.335989 85.316989) (end 134.886 85.867) (width 0.2) (layer F.Cu) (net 5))
 (segment (start 134.886 85.867) (end 135.761 85.867) (width 0.2) (layer F.Cu) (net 5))
 (segment (start 134.335989 81.651687) (end 134.335989 85.316989) (width 0.2) (layer F.Cu) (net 5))
 (segment (start 133.194302 80.51) (end 134.335989 81.651687) (width 0.2) (layer F.Cu) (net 5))
 (segment (start 132.31 80.51) (end 133.194302 80.51) (width 0.2) (layer F.Cu) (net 5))
 (segment (start 123.063 79.144) (end 123.04 79.121) (width 0.25) (layer B.Cu) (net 1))
 (segment (start 123.04 80.972002) (end 123.063 80.995002) (width 0.25) (layer B.Cu) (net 1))
 (segment (start 123.04 79.121) (end 123.04 80.972002) (width 0.25) (layer B.Cu) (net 1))
 (segment (start 123.04 79.121) (end 124.379 79.121) (width 0.25) (layer B.Cu) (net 1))
 (via (at 124.206 83.312) (size 0.8) (drill 0.4) (layers F.Cu B.Cu) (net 2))
 (segment (start 124.206 83.312) (end 124.206 83.877685) (width 0.25) (layer F.Cu) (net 2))
 (segment (start 124.783315 84.455) (end 133.179 84.455) (width 0.25) (layer F.Cu) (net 2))
 (segment (start 124.206 83.877685) (end 124.783315 84.455) (width 0.25) (layer F.Cu) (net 2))
 (segment (start 124.333 79.167) (end 124.379 79.121) (width 0.25) (layer F.Cu) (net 11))
 (segment (start 124.333 80.995002) (end 124.333 79.167) (width 0.25) (layer F.Cu) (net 11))
 (segment (start 126.779 83.305) (end 127.679 83.305) (width 0.25) (layer F.Cu) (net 11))
 (segment (start 126.417591 83.305) (end 126.779 83.305) (width 0.25) (layer F.Cu) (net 11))
 (segment (start 124.658 81.320002) (end 124.658 81.545409) (width 0.25) (layer F.Cu) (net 11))
 (segment (start 124.658 81.545409) (end 126.417591 83.305) (width 0.25) (layer F.Cu) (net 11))
 (segment (start 124.333 80.995002) (end 124.658 81.320002) (width 0.25) (layer F.Cu) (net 11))
 (segment (start 123.806001 83.711999) (end 124.206 83.312) (width 0.25) (layer F.Cu) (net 2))
 (segment (start 123.388 84.13) (end 123.806001 83.711999) (width 0.25) (layer F.Cu) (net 2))
 (segment (start 123.388 86.320001) (end 123.388 84.13) (width 0.25) (layer F.Cu) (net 2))
 (segment (start 123.063 86.645001) (end 123.388 86.320001) (width 0.25) (layer F.Cu) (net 2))
 (via (at 125.349 78.0415) (size 0.8) (drill 0.4) (layers F.Cu B.Cu) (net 2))
 (segment (start 125.349 79.121) (end 125.349 78.0415) (width 0.25) (layer B.Cu) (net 2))
 (segment (start 124.206 79.1845) (end 124.206 83.312) (width 0.5) (layer v33) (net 2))
 (segment (start 125.349 78.0415) (end 124.206 79.1845) (width 0.5) (layer v33) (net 2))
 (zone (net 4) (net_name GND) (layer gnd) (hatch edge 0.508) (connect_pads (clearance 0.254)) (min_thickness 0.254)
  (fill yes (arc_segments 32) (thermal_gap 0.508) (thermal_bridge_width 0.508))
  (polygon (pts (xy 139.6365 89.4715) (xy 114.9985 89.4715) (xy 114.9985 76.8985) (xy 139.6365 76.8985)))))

